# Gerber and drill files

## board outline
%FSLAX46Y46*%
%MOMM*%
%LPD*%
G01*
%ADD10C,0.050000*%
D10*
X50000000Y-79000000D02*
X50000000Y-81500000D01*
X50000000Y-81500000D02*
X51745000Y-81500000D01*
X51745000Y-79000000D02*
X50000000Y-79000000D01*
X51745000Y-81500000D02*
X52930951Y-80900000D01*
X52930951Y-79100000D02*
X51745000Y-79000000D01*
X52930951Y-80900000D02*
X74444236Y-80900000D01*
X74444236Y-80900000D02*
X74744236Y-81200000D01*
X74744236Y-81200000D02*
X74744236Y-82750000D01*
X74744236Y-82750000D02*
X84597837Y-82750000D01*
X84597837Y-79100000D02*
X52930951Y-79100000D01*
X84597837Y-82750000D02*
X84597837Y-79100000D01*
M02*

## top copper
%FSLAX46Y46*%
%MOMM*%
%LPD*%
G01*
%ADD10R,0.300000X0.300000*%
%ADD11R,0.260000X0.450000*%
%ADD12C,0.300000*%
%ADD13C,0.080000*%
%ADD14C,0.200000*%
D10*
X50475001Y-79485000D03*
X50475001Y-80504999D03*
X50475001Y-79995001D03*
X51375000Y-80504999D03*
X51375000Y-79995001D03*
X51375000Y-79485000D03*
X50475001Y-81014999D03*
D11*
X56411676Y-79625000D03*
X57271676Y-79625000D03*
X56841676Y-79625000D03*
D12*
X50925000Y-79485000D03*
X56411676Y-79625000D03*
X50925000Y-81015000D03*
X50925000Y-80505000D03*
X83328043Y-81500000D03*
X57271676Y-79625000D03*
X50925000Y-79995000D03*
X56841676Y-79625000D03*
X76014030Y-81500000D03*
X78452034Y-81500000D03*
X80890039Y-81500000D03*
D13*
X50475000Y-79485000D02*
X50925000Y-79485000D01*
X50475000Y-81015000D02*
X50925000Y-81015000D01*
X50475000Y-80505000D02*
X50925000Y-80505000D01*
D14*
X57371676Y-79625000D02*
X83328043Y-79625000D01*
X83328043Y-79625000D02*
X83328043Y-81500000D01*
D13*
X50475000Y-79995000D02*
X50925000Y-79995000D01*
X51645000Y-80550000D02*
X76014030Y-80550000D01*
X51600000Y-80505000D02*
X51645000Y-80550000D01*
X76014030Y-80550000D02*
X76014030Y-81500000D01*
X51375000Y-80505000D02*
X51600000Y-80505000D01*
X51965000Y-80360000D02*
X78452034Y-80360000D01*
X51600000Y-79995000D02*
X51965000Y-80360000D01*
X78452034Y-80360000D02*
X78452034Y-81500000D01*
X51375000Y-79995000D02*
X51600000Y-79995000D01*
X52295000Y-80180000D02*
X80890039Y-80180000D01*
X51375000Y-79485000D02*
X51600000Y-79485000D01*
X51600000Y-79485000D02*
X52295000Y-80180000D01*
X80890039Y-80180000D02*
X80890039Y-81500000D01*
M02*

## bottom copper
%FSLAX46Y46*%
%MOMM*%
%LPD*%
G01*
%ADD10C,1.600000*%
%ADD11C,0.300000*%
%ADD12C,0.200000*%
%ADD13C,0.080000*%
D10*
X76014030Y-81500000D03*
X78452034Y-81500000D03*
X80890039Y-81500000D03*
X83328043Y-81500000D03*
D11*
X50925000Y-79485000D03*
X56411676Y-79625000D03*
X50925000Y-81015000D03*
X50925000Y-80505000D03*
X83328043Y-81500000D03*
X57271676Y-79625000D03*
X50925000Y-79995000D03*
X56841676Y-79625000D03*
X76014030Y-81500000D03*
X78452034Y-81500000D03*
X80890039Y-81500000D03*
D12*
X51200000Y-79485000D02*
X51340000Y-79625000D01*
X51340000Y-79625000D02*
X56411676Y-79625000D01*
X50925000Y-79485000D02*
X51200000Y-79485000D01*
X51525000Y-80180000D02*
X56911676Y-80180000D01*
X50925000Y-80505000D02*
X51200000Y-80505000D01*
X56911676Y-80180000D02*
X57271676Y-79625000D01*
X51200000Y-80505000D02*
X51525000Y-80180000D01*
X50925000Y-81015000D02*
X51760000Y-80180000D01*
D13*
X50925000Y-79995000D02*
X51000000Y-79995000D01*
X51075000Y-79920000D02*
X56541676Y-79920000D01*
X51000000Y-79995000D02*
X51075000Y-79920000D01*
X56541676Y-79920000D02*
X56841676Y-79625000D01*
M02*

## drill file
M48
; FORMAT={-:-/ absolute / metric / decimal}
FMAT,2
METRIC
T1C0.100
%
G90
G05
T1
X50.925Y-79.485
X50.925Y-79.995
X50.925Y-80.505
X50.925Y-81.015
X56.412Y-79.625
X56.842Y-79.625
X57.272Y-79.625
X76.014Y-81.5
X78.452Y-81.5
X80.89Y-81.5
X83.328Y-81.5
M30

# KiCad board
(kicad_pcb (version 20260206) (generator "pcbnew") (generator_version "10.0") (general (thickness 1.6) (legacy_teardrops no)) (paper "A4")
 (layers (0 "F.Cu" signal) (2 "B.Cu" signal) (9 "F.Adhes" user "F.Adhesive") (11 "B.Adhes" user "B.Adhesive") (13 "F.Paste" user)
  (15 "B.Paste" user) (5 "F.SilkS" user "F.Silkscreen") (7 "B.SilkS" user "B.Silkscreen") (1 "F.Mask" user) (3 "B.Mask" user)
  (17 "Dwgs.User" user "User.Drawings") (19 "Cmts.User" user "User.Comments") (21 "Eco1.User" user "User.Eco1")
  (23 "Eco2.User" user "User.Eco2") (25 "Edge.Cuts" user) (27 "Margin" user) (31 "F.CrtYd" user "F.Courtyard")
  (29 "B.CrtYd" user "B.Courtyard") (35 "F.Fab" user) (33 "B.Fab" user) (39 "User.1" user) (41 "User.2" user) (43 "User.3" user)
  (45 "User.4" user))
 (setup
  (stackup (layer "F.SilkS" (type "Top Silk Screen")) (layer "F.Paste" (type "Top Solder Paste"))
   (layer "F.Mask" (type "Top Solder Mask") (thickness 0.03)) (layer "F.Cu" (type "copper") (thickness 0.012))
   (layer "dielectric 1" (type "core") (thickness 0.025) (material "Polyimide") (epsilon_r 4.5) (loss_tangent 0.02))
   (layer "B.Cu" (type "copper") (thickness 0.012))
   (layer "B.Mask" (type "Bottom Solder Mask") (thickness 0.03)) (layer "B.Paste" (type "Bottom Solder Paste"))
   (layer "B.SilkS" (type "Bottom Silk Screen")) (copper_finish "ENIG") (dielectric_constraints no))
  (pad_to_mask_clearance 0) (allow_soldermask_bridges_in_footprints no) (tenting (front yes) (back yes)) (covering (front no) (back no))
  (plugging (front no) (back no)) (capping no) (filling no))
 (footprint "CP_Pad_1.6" (layer "F.Cu") (at 76.01403 81.5)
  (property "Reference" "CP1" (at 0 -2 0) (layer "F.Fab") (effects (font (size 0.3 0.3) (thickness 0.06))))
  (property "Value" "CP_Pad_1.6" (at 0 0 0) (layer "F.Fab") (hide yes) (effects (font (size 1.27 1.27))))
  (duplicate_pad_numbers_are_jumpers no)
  (pad "1" smd circle (at 0 0) (size 1.6 1.6) (layers "B.Cu" "B.Mask") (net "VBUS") (solder_mask_margin 0.1)))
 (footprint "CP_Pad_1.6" (layer "F.Cu") (at 83.328043 81.5)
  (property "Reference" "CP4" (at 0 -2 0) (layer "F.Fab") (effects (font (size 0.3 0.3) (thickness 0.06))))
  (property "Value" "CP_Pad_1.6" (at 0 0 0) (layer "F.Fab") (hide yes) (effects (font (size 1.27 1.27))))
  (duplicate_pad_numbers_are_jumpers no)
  (pad "1" smd circle (at 0 0) (size 1.6 1.6) (layers "B.Cu" "B.Mask") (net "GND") (solder_mask_margin 0.1)))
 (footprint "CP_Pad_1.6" (layer "F.Cu") (at 80.890039 81.5)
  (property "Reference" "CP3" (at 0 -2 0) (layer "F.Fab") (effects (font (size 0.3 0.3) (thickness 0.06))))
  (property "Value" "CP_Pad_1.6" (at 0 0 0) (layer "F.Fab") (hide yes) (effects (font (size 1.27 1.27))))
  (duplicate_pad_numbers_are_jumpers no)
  (pad "1" smd circle (at 0 0) (size 1.6 1.6) (layers "B.Cu" "B.Mask") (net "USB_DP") (solder_mask_margin 0.1)))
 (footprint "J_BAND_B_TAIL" (layer "F.Cu") (at 50.9 80.25)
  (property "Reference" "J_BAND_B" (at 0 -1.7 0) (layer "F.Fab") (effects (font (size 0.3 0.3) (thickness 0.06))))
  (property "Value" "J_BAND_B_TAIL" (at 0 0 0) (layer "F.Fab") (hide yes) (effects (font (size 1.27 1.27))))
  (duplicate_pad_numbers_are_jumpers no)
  (pad "1" smd rect (at -0.424999 -0.765) (size 0.3 0.3) (layers "F.Cu" "F.Mask") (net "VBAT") (solder_mask_margin 0.05)
   (thermal_bridge_angle 45))
  (pad "2" smd rect (at -0.424999 0.254999) (size 0.3 0.3) (layers "F.Cu" "F.Mask") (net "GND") (solder_mask_margin 0.05)
   (thermal_bridge_angle 45))
  (pad "3" smd rect (at -0.424999 -0.254999) (size 0.3 0.3) (layers "F.Cu" "F.Mask") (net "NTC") (solder_mask_margin 0.05)
   (thermal_bridge_angle 45))
  (pad "4" smd rect (at 0.475 0.254999) (size 0.3 0.3) (layers "F.Cu" "F.Mask") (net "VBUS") (solder_mask_margin 0.05)
   (thermal_bridge_angle 45))
  (pad "5" smd rect (at 0.475 -0.254999) (size 0.3 0.3) (layers "F.Cu" "F.Mask") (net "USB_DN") (solder_mask_margin 0.05)
   (thermal_bridge_angle 45))
  (pad "6" smd rect (at 0.475 -0.765) (size 0.3 0.3) (layers "F.Cu" "F.Mask") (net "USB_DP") (solder_mask_margin 0.05)
   (thermal_bridge_angle 45))
  (pad "7" smd rect (at -0.424999 0.764999) (size 0.3 0.3) (layers "F.Cu" "F.Mask") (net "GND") (solder_mask_margin 0.05)
   (thermal_bridge_angle 45)))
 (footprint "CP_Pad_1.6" (layer "F.Cu") (at 78.452034 81.5)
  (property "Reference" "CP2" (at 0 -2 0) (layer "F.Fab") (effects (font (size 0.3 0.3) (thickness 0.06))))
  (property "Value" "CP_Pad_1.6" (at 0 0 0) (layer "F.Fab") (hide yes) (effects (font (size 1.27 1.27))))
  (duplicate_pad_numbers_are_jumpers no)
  (pad "1" smd circle (at 0 0) (size 1.6 1.6) (layers "B.Cu" "B.Mask") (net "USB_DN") (solder_mask_margin 0.1)))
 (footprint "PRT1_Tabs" (layer "F.Cu") (at 56.841676 79.625)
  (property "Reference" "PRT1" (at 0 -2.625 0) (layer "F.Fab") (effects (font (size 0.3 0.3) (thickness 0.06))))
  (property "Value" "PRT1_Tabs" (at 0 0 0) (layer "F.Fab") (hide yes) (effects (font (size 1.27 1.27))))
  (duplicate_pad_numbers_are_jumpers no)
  (pad "1" smd rect (at -0.43 0) (size 0.26 0.45) (layers "F.Cu" "F.Mask") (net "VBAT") (solder_mask_margin 0.05) (thermal_bridge_angle 45))
  (pad "2" smd rect (at 0.43 0) (size 0.26 0.45) (layers "F.Cu" "F.Mask") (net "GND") (solder_mask_margin 0.05) (thermal_bridge_angle 45))
  (pad "3" smd rect (at 0 0) (size 0.26 0.45) (layers "F.Cu" "F.Mask") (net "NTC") (solder_mask_margin 0.05) (thermal_bridge_angle 45)))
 (gr_line (start 50 79) (end 50 81.5) (stroke (width 0.05) (type default)) (layer "Edge.Cuts"))
 (gr_line (start 50 81.5) (end 51.745 81.5) (stroke (width 0.05) (type default)) (layer "Edge.Cuts"))
 (gr_line (start 51.745 79) (end 50 79) (stroke (width 0.05) (type default)) (layer "Edge.Cuts"))
 (gr_line (start 51.745 81.5) (end 52.930951 80.9) (stroke (width 0.05) (type default)) (layer "Edge.Cuts"))
 (gr_line (start 52.930951 79.1) (end 51.745 79) (stroke (width 0.05) (type default)) (layer "Edge.Cuts"))
 (gr_line (start 52.930951 80.9) (end 74.444236 80.9) (stroke (width 0.05) (type default)) (layer "Edge.Cuts"))
 (gr_line (start 74.444236 80.9) (end 74.744236 81.2) (stroke (width 0.05) (type default)) (layer "Edge.Cuts"))
 (gr_line (start 74.744236 81.2) (end 74.744236 82.75) (stroke (width 0.05) (type default)) (layer "Edge.Cuts"))
 (gr_line (start 74.744236 82.75) (end 84.597837 82.75) (stroke (width 0.05) (type default)) (layer "Edge.Cuts"))
 (gr_line (start 84.597837 79.1) (end 52.930951 79.1) (stroke (width 0.05) (type default)) (layer "Edge.Cuts"))
 (gr_line (start 84.597837 82.75) (end 84.597837 79.1) (stroke (width 0.05) (type default)) (layer "Edge.Cuts"))
 (segment (start 51.375 80.505) (end 51.6 80.505) (width 0.08) (layer "F.Cu") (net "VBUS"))
 (segment (start 51.645 80.55) (end 76.01403 80.55) (width 0.08) (layer "F.Cu") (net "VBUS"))
 (segment (start 76.01403 80.55) (end 76.01403 81.5) (width 0.08) (layer "F.Cu") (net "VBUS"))
 (segment (start 51.6 80.505) (end 51.645 80.55) (width 0.08) (layer "F.Cu") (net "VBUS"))
 (via (at 76.01403 81.5) (size 0.3) (drill 0.1) (layers "F.Cu" "B.Cu") (tenting (front yes) (back yes)) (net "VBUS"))
 (segment (start 57.371676 79.625) (end 83.328043 79.625) (width 0.2) (layer "F.Cu") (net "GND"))
 (segment (start 50.475 81.015) (end 50.925 81.015) (width 0.08) (layer "F.Cu") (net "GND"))
 (segment (start 50.475 80.505) (end 50.925 80.505) (width 0.08) (layer "F.Cu") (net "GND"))
 (segment (start 83.328043 79.625) (end 83.328043 81.5) (width 0.2) (layer "F.Cu") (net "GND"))
 (via (at 57.271676 79.625) (size 0.3) (drill 0.1) (layers "F.Cu" "B.Cu") (tenting (front yes) (back yes)) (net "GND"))
 (via (at 50.925 80.505) (size 0.3) (drill 0.1) (layers "F.Cu" "B.Cu") (tenting (front yes) (back yes)) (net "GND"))
 (via (at 50.925 81.015) (size 0.3) (drill 0.1) (layers "F.Cu" "B.Cu") (tenting (front yes) (back yes)) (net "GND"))
 (via (at 83.328043 81.5) (size 0.3) (drill 0.1) (layers "F.Cu" "B.Cu") (tenting (front yes) (back yes)) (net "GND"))
 (segment (start 50.925 80.505) (end 51.2 80.505) (width 0.2) (layer "B.Cu") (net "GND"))
 (segment (start 51.525 80.18) (end 56.911676 80.18) (width 0.2) (layer "B.Cu") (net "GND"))
 (segment (start 51.2 80.505) (end 51.525 80.18) (width 0.2) (layer "B.Cu") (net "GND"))
 (segment (start 56.911676 80.18) (end 57.271676 79.625) (width 0.2) (layer "B.Cu") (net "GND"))
 (segment (start 50.925 81.015) (end 51.76 80.18) (width 0.2) (layer "B.Cu") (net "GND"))
 (segment (start 52.295 80.18) (end 80.890039 80.18) (width 0.08) (layer "F.Cu") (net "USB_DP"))
 (segment (start 51.6 79.485) (end 52.295 80.18) (width 0.08) (layer "F.Cu") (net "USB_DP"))
 (segment (start 80.890039 80.18) (end 80.890039 81.5) (width 0.08) (layer "F.Cu") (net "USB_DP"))
 (segment (start 51.375 79.485) (end 51.6 79.485) (width 0.08) (layer "F.Cu") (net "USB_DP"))
 (via (at 80.890039 81.5) (size 0.3) (drill 0.1) (layers "F.Cu" "B.Cu") (tenting (front yes) (back yes)) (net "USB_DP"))
 (segment (start 50.475 79.485) (end 51.025 79.485) (width 0.08) (layer "F.Cu") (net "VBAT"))
 (via (at 50.925 79.485) (size 0.3) (drill 0.1) (layers "F.Cu" "B.Cu") (tenting (front yes) (back yes)) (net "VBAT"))
 (via (at 56.411676 79.625) (size 0.3) (drill 0.1) (layers "F.Cu" "B.Cu") (tenting (front yes) (back yes)) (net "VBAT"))
 (segment (start 50.925 79.485) (end 51.2 79.485) (width 0.2) (layer "B.Cu") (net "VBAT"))
 (segment (start 51.34 79.625) (end 56.411676 79.625) (width 0.2) (layer "B.Cu") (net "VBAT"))
 (segment (start 51.2 79.485) (end 51.34 79.625) (width 0.2) (layer "B.Cu") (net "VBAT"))
 (segment (start 50.475 79.995) (end 50.925 79.995) (width 0.08) (layer "F.Cu") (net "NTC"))
 (via (at 50.925 79.995) (size 0.3) (drill 0.1) (layers "F.Cu" "B.Cu") (tenting (front yes) (back yes)) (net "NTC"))
 (via (at 56.841676 79.625) (size 0.3) (drill 0.1) (layers "F.Cu" "B.Cu") (tenting (front yes) (back yes)) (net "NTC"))
 (segment (start 51 79.995) (end 51.075 79.92) (width 0.08) (layer "B.Cu") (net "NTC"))
 (segment (start 56.541676 79.92) (end 56.841676 79.625) (width 0.08) (layer "B.Cu") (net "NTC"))
 (segment (start 51.075 79.92) (end 56.541676 79.92) (width 0.08) (layer "B.Cu") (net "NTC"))
 (segment (start 50.925 79.995) (end 51 79.995) (width 0.08) (layer "B.Cu") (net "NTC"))
 (segment (start 51.375 79.995) (end 51.6 79.995) (width 0.08) (layer "F.Cu") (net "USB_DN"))
 (segment (start 51.6 79.995) (end 51.965 80.36) (width 0.08) (layer "F.Cu") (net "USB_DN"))
 (segment (start 51.965 80.36) (end 78.452034 80.36) (width 0.08) (layer "F.Cu") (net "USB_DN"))
 (segment (start 78.452034 80.36) (end 78.452034 81.5) (width 0.08) (layer "F.Cu") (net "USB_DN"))
 (via (at 78.452034 81.5) (size 0.3) (drill 0.1) (layers "F.Cu" "B.Cu") (tenting (front yes) (back yes)) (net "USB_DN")))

